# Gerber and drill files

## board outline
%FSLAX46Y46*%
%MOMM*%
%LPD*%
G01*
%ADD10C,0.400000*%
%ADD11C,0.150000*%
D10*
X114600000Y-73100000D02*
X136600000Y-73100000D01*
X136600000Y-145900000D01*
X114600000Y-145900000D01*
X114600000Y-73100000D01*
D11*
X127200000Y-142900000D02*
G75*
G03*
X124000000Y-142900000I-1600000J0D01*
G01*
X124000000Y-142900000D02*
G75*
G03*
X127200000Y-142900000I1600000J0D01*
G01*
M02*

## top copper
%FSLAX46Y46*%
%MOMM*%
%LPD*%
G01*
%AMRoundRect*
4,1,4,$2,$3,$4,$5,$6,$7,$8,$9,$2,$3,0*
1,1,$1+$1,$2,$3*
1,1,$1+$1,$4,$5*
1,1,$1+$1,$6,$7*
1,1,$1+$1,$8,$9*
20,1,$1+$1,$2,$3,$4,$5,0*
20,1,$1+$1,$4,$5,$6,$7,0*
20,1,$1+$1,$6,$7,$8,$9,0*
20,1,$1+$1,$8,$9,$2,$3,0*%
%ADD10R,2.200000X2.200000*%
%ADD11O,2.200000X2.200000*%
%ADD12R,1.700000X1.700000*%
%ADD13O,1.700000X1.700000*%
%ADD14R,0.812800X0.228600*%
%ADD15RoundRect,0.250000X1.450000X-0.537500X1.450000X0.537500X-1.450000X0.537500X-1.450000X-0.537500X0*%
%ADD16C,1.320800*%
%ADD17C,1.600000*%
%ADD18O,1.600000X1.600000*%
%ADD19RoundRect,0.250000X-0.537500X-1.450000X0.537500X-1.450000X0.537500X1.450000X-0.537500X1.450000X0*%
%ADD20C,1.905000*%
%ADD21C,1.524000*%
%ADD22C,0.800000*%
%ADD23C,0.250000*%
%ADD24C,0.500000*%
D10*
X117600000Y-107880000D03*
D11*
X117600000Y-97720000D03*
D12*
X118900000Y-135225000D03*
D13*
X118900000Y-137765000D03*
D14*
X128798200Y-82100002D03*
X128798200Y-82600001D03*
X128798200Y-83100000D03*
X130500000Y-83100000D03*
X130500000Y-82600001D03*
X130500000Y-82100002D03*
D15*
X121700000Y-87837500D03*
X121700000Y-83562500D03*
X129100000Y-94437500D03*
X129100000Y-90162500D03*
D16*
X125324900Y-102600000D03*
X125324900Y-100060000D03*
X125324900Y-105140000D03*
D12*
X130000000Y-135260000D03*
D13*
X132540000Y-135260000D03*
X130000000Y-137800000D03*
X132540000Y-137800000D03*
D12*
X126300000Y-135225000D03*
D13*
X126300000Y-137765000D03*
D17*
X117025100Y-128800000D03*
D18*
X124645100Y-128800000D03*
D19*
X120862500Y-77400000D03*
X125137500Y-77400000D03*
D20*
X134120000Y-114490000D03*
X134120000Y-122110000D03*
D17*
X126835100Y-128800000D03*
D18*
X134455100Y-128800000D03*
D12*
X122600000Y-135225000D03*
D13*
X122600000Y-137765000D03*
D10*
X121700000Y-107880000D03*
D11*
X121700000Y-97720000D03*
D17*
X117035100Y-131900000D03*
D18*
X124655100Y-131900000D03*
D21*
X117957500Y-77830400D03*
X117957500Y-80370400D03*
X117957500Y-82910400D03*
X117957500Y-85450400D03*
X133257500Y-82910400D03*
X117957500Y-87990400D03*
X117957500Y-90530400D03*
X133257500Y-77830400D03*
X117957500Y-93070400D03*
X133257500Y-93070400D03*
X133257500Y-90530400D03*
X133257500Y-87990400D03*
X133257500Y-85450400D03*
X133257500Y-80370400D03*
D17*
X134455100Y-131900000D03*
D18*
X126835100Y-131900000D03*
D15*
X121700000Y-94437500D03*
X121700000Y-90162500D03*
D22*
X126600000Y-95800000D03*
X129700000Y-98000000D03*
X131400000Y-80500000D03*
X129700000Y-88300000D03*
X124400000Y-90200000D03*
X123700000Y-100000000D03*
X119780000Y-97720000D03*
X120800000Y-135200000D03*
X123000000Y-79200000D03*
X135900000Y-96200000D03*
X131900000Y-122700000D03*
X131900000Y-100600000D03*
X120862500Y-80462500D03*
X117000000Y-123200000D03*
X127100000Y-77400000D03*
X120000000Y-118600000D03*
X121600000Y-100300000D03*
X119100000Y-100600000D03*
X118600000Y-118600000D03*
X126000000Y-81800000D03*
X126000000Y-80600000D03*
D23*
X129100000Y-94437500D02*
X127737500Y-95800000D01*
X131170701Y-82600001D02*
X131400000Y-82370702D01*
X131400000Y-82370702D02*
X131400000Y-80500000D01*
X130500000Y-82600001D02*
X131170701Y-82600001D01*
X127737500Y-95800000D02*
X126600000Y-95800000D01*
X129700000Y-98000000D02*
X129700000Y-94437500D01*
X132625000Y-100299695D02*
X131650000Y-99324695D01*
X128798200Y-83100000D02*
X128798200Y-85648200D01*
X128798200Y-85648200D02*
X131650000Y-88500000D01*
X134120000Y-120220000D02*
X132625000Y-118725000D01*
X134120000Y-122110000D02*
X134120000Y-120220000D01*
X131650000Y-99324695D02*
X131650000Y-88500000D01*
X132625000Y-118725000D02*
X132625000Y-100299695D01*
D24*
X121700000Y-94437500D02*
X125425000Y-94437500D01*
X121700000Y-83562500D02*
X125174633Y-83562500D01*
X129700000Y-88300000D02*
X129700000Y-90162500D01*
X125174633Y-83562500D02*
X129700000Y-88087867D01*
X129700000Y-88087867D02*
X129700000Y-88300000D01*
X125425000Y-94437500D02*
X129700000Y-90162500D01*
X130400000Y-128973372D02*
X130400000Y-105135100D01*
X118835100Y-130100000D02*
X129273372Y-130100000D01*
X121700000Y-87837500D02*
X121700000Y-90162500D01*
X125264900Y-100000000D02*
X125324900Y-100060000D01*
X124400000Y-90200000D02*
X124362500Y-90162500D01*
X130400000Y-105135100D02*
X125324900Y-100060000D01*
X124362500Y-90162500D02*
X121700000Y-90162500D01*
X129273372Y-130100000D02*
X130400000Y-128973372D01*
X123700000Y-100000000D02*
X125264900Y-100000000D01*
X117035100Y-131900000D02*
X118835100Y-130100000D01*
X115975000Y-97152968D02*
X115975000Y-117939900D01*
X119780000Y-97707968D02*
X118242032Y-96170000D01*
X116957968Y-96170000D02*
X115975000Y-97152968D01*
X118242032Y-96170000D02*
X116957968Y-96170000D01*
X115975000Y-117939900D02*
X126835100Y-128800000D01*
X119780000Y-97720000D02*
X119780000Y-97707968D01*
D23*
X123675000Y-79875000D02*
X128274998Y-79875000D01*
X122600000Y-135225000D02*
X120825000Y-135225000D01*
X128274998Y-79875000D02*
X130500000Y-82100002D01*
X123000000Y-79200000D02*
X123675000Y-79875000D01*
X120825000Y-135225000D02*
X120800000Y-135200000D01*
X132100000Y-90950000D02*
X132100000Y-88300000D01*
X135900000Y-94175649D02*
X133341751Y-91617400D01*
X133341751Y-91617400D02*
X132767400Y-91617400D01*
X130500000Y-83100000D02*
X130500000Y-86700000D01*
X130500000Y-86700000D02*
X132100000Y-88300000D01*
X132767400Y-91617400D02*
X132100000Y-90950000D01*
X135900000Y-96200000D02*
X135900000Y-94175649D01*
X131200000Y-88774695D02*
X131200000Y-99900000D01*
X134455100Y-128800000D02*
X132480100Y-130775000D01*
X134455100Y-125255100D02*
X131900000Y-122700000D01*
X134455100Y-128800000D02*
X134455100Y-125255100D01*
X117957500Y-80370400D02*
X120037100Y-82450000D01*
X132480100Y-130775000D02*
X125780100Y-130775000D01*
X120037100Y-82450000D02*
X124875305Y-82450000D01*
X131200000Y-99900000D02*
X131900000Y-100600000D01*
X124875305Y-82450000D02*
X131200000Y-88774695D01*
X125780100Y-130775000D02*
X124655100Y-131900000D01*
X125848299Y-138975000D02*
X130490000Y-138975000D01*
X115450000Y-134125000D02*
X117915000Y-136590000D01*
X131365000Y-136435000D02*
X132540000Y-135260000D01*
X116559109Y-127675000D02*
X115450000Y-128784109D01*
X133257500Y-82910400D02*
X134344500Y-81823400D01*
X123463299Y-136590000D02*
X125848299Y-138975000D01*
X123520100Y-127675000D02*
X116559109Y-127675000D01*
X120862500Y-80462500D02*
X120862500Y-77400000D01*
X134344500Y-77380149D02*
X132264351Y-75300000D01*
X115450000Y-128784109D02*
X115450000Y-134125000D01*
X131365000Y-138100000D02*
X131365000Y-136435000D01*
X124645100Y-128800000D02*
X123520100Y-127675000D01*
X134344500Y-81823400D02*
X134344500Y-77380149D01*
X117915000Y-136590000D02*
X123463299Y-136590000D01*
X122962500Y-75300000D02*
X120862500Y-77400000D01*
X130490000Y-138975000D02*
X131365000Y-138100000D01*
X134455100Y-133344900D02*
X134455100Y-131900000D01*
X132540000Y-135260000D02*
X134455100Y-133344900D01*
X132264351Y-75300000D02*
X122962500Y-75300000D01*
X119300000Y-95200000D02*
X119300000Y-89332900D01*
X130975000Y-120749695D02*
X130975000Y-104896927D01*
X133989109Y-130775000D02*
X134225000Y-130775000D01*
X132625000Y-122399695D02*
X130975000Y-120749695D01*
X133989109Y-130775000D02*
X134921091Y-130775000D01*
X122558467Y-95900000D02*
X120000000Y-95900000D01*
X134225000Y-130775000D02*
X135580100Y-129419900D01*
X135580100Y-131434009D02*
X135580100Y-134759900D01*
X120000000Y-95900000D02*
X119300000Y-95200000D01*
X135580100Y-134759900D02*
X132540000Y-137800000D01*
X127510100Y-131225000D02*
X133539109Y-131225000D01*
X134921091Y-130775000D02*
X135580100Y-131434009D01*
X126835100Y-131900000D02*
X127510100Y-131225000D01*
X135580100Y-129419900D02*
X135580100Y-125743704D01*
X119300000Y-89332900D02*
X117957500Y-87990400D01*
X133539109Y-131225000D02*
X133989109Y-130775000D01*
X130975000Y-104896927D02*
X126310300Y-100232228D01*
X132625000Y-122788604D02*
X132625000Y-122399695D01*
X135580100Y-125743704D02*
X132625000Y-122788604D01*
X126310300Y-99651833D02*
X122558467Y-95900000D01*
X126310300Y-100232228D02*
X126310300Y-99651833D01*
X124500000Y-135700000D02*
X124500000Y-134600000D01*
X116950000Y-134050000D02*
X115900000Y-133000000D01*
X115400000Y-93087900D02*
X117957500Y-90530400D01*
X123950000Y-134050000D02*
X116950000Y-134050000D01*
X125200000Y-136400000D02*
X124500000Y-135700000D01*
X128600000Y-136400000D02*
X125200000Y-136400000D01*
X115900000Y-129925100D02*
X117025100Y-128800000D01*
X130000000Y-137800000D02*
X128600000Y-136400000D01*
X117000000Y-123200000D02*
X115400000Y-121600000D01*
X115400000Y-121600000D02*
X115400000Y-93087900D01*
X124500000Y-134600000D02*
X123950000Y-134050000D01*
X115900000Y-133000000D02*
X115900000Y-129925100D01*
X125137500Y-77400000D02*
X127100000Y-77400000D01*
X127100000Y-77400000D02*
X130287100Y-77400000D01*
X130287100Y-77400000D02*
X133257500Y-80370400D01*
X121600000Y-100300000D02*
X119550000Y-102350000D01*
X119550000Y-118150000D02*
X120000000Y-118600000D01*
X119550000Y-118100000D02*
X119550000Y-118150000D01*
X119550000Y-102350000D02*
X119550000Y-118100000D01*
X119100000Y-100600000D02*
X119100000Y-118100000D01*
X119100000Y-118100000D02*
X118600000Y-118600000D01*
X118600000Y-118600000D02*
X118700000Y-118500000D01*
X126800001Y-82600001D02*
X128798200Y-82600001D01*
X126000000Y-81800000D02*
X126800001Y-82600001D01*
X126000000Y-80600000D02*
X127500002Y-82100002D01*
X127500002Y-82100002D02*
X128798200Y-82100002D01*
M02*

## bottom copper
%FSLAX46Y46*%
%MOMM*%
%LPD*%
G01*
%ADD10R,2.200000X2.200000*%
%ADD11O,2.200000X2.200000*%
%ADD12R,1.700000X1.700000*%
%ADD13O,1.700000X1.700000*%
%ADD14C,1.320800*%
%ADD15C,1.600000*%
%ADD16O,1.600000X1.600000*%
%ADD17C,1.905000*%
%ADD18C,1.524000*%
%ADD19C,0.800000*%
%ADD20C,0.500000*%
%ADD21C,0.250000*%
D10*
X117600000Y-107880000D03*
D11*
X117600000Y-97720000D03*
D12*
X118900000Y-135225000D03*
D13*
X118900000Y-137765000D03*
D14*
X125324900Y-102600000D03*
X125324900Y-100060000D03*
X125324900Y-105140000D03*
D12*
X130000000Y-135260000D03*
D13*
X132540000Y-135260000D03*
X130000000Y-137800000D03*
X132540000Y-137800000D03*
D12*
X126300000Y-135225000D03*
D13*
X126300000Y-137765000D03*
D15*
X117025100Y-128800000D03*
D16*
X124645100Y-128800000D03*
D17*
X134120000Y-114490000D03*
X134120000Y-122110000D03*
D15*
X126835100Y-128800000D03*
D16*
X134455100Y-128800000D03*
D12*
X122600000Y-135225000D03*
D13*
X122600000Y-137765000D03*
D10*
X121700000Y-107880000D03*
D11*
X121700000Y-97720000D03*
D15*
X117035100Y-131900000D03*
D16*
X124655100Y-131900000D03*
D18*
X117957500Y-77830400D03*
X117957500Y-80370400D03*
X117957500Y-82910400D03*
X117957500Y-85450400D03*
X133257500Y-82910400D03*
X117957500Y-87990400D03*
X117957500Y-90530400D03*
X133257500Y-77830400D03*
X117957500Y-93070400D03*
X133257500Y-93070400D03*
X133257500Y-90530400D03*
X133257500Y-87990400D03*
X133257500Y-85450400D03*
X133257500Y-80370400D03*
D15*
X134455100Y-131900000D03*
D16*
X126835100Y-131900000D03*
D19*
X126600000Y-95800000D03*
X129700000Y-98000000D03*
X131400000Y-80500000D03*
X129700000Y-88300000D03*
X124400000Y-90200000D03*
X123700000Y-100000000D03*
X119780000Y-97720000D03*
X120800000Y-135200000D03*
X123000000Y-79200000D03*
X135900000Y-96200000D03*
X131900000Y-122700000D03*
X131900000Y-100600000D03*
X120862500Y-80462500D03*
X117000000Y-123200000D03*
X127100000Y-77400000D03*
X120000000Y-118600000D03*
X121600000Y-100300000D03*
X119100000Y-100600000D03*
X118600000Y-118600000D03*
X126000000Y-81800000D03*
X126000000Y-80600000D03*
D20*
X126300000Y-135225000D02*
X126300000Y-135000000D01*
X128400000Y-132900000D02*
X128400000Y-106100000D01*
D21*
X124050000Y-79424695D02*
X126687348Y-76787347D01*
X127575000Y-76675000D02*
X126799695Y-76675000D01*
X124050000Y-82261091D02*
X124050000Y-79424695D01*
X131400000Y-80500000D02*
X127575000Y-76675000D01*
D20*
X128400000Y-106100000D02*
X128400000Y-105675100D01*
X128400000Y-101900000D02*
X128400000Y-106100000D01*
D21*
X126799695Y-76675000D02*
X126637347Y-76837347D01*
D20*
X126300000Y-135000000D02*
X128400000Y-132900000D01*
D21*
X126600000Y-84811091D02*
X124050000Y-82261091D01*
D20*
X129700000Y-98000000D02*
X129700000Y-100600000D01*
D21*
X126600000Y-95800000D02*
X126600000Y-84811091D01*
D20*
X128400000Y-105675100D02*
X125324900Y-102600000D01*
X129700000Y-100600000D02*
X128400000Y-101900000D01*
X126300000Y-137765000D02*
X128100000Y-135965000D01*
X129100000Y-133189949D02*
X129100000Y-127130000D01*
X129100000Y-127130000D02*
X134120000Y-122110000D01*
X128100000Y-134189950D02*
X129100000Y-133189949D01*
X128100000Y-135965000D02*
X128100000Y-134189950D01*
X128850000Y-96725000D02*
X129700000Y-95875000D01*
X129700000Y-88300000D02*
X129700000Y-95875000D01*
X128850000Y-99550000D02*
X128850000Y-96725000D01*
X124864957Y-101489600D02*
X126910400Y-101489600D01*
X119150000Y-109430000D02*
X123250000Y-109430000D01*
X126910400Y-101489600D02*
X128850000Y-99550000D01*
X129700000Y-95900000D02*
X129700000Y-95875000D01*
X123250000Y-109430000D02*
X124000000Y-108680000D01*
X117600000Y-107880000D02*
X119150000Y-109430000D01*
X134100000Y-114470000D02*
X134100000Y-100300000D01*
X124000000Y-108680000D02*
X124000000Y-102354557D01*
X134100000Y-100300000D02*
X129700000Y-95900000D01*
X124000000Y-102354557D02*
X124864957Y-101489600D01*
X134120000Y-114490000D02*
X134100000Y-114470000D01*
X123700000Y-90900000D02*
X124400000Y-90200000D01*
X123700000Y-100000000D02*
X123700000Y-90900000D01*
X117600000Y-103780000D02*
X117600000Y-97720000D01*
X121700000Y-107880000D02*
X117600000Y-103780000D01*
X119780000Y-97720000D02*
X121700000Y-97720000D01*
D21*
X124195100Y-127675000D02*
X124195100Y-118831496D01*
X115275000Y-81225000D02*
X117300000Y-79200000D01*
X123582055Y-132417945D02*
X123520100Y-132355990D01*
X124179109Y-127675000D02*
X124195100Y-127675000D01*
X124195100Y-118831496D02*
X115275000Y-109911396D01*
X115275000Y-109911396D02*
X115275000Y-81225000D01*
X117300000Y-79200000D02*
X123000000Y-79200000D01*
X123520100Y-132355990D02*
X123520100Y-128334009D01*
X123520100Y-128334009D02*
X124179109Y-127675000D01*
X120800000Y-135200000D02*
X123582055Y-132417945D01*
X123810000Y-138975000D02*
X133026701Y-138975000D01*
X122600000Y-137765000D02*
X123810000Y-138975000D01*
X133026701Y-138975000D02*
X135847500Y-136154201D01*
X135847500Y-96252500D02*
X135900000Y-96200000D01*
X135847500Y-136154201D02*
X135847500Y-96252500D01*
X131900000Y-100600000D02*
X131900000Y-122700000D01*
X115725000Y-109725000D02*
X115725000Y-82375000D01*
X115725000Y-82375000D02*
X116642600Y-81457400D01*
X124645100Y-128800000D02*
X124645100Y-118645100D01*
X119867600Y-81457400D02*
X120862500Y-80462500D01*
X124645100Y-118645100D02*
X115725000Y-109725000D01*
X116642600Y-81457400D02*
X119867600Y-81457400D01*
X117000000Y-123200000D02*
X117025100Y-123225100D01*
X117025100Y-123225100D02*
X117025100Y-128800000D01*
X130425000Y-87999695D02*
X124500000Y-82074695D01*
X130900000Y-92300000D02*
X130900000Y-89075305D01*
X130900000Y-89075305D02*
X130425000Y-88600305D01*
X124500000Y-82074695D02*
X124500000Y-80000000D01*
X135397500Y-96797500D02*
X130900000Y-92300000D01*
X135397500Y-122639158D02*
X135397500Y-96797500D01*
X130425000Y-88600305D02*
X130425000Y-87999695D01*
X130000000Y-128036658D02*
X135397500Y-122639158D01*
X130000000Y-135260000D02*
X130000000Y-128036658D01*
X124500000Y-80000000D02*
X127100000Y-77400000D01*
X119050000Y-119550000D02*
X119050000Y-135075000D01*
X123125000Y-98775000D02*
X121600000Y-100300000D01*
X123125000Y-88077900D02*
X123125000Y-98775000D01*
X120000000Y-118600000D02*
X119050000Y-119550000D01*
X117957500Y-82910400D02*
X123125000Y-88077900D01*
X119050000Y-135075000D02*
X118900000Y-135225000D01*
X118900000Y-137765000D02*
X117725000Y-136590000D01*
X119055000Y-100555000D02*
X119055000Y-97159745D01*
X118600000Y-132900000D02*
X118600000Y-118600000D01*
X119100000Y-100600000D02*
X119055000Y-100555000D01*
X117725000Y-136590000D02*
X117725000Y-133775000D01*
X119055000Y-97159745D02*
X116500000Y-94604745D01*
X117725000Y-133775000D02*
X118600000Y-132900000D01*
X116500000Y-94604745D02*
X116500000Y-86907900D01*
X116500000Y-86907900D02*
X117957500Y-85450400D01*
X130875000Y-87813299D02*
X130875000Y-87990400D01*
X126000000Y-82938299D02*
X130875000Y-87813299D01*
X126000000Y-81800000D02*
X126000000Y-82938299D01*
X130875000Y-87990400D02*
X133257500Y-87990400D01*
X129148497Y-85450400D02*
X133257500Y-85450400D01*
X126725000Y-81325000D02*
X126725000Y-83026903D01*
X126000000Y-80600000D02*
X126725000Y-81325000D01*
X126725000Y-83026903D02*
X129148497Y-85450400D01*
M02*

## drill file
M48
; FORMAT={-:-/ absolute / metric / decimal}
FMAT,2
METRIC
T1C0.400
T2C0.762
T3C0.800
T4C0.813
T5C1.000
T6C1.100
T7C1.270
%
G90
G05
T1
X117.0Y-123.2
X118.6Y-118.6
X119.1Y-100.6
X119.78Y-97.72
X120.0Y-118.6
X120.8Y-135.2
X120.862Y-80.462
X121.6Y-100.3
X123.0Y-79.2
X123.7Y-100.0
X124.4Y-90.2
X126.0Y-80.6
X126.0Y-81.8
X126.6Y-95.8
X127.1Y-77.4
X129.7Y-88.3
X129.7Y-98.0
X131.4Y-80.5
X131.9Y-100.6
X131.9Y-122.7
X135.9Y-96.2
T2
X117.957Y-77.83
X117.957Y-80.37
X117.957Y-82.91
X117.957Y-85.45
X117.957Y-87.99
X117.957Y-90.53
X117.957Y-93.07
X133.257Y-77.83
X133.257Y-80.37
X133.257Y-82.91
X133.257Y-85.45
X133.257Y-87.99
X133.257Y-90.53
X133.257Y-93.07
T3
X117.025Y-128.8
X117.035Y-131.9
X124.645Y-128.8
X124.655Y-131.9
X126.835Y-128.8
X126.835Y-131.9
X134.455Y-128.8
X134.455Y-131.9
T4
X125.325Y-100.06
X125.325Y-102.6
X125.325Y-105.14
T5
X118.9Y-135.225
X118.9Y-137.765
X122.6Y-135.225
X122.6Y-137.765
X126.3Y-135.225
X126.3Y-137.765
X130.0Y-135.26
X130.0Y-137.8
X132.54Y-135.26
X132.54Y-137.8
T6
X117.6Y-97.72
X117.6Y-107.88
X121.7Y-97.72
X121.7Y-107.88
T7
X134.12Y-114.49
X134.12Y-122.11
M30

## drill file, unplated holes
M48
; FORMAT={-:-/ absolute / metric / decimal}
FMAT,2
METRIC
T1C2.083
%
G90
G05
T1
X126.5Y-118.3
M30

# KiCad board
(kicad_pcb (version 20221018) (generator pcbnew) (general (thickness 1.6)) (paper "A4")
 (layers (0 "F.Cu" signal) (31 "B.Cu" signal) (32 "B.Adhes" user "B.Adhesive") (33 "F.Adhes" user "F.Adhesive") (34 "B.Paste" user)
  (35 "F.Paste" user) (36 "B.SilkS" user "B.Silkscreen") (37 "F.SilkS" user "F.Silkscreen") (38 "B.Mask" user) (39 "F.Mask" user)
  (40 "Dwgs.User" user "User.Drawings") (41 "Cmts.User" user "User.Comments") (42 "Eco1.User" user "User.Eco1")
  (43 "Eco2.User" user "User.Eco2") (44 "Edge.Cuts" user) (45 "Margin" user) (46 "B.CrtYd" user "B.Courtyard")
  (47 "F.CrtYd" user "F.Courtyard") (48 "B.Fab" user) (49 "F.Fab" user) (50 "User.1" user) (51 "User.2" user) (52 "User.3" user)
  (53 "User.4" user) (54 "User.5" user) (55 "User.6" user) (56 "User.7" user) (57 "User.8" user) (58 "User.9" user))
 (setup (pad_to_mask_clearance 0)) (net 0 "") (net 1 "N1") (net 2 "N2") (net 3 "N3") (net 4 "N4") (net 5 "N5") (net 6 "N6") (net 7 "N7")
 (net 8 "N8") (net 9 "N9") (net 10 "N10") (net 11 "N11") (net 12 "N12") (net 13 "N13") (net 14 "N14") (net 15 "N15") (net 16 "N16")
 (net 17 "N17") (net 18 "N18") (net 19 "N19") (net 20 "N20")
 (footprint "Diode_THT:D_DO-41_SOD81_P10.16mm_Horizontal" (layer "F.Cu") (at 117.6 107.88 90)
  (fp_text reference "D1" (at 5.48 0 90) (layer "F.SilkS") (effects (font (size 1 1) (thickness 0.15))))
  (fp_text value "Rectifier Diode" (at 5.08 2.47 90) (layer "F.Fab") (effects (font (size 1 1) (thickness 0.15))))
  (pad "1" thru_hole rect (at 0 0 90) (size 2.2 2.2) (drill 1.1) (layers "*.Cu" "*.Mask") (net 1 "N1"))
  (pad "2" thru_hole oval (at 10.16 0 90) (size 2.2 2.2) (drill 1.1) (layers "*.Cu" "*.Mask") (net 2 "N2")))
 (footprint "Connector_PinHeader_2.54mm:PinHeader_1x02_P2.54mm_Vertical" (layer "F.Cu") (at 118.9 135.225)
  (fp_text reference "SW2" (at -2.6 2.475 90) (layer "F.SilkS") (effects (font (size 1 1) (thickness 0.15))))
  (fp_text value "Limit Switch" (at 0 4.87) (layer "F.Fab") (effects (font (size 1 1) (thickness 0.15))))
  (pad "1" thru_hole rect (at 0 0) (size 1.7 1.7) (drill 1) (layers "*.Cu" "*.Mask") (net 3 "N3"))
  (pad "2" thru_hole oval (at 0 2.54) (size 1.7 1.7) (drill 1) (layers "*.Cu" "*.Mask") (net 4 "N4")))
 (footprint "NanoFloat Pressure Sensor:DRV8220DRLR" (layer "F.Cu") (at 129.6491 82.600001)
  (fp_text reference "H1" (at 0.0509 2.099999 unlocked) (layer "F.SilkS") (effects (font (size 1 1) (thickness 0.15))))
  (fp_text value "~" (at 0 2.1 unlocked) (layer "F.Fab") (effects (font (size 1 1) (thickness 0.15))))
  (pad "1" smd rect (at -0.8509 -0.499999) (size 0.8128 0.2286) (layers "F.Cu" "F.Paste" "F.Mask") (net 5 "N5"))
  (pad "2" smd rect (at -0.8509 0) (size 0.8128 0.2286) (layers "F.Cu" "F.Paste" "F.Mask") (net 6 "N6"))
  (pad "3" smd rect (at -0.8509 0.499999) (size 0.8128 0.2286) (layers "F.Cu" "F.Paste" "F.Mask") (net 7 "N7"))
  (pad "4" smd rect (at 0.8509 0.499999) (size 0.8128 0.2286) (layers "F.Cu" "F.Paste" "F.Mask") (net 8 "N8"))
  (pad "5" smd rect (at 0.8509 0) (size 0.8128 0.2286) (layers "F.Cu" "F.Paste" "F.Mask") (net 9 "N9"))
  (pad "6" smd rect (at 0.8509 -0.499999) (size 0.8128 0.2286) (layers "F.Cu" "F.Paste" "F.Mask") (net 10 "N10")))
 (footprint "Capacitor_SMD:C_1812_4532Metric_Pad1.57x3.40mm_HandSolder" (layer "F.Cu") (at 121.7 85.7 90)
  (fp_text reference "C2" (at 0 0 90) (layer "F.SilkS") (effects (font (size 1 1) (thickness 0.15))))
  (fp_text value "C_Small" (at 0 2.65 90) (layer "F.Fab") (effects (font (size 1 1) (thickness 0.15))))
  (pad "1" smd roundrect (at -2.1375 0 90) (size 1.575 3.4) (layers "F.Cu" "F.Paste" "F.Mask") (roundrect_rratio 0.1587301587)
   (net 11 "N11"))
  (pad "2" smd roundrect (at 2.1375 0 90) (size 1.575 3.4) (layers "F.Cu" "F.Paste" "F.Mask") (roundrect_rratio 0.1587301587) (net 1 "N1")))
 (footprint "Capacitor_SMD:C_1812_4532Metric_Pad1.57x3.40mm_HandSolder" (layer "F.Cu") (at 129.1 92.3 90)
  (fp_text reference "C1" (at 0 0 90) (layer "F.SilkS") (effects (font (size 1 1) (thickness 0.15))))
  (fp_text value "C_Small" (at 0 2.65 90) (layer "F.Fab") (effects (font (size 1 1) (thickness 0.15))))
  (pad "1" smd roundrect (at -2.1375 0 90) (size 1.575 3.4) (layers "F.Cu" "F.Paste" "F.Mask") (roundrect_rratio 0.1587301587) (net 9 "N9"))
  (pad "2" smd roundrect (at 2.1375 0 90) (size 1.575 3.4) (layers "F.Cu" "F.Paste" "F.Mask") (roundrect_rratio 0.1587301587) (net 1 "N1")))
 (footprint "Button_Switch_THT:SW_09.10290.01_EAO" (layer "F.Cu") (at 125.3249 102.6 90)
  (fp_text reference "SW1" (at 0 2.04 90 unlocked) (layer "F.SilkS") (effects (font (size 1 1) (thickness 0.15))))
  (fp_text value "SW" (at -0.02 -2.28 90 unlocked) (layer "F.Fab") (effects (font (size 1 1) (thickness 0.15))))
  (pad "1" thru_hole circle (at 0 0 90) (size 1.3208 1.3208) (drill 0.8128) (layers "*.Cu" "*.Mask") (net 9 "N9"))
  (pad "2" thru_hole circle (at 2.54 0 90) (size 1.3208 1.3208) (drill 0.8128) (layers "*.Cu" "*.Mask") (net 11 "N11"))
  (pad "3" thru_hole circle (at -2.54 0 90) (size 1.3208 1.3208) (drill 0.8128) (layers "*.Cu" "*.Mask") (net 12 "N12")))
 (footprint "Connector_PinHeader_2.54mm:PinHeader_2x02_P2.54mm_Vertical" (layer "F.Cu") (at 130 135.26)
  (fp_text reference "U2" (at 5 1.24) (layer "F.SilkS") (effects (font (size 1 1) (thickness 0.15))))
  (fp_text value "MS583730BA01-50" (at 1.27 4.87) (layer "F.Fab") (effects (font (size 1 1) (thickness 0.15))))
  (pad "1" thru_hole rect (at 0 0) (size 1.7 1.7) (drill 1) (layers "*.Cu" "*.Mask") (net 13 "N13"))
  (pad "2" thru_hole oval (at 2.54 0) (size 1.7 1.7) (drill 1) (layers "*.Cu" "*.Mask") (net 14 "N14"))
  (pad "3" thru_hole oval (at 0 2.54) (size 1.7 1.7) (drill 1) (layers "*.Cu" "*.Mask") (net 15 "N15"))
  (pad "4" thru_hole oval (at 2.54 2.54) (size 1.7 1.7) (drill 1) (layers "*.Cu" "*.Mask") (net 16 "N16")))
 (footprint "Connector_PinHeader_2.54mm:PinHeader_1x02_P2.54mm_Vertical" (layer "F.Cu") (at 126.3 135.225)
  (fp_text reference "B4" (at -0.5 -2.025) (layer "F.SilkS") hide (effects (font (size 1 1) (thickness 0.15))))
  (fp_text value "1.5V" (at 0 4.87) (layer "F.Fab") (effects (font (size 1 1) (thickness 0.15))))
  (pad "1" thru_hole rect (at 0 0) (size 1.7 1.7) (drill 1) (layers "*.Cu" "*.Mask") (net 9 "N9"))
  (pad "2" thru_hole oval (at 0 2.54) (size 1.7 1.7) (drill 1) (layers "*.Cu" "*.Mask") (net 7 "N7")))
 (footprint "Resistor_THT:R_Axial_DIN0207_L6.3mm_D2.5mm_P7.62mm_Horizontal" (layer "F.Cu") (at 117.0251 128.8)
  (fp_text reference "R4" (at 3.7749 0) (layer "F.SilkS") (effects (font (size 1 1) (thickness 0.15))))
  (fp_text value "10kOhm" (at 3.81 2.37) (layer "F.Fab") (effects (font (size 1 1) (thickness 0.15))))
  (pad "1" thru_hole circle (at 0 0) (size 1.6 1.6) (drill 0.8) (layers "*.Cu" "*.Mask") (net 15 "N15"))
  (pad "2" thru_hole oval (at 7.62 0) (size 1.6 1.6) (drill 0.8) (layers "*.Cu" "*.Mask") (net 14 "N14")))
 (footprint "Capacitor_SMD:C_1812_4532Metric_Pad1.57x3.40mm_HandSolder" (layer "F.Cu") (at 123 77.4)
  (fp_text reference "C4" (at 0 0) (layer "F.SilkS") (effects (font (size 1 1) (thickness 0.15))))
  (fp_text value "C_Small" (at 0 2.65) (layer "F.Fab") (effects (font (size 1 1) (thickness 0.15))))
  (pad "1" smd roundrect (at -2.1375 0) (size 1.575 3.4) (layers "F.Cu" "F.Paste" "F.Mask") (roundrect_rratio 0.1587301587) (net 14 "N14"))
  (pad "2" smd roundrect (at 2.1375 0) (size 1.575 3.4) (layers "F.Cu" "F.Paste" "F.Mask") (roundrect_rratio 0.1587301587) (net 13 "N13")))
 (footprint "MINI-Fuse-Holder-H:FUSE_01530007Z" (layer "F.Cu") (at 126.5 118.3 -90)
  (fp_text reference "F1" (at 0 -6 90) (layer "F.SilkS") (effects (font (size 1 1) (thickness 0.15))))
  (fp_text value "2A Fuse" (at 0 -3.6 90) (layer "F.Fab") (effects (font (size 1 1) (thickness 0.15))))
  (pad "" np_thru_hole circle (at 0 0 270) (size 2.0828 2.0828) (drill 2.0828) (layers "*.Cu" "*.Mask"))
  (pad "1" thru_hole circle (at -3.81 -7.62 270) (size 1.905 1.905) (drill 1.27) (layers "*.Cu" "*.Mask") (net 1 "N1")
   (solder_mask_margin 0.102))
  (pad "2" thru_hole circle (at 3.81 -7.62 270) (size 1.905 1.905) (drill 1.27) (layers "*.Cu" "*.Mask") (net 7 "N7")
   (solder_mask_margin 0.102)))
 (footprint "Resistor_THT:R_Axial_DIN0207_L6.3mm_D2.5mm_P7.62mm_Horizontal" (layer "F.Cu") (at 126.8351 128.8)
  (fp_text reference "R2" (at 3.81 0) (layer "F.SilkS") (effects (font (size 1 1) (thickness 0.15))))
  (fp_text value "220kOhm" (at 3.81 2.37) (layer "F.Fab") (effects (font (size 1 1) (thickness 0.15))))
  (pad "1" thru_hole circle (at 0 0) (size 1.6 1.6) (drill 0.8) (layers "*.Cu" "*.Mask") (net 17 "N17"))
  (pad "2" thru_hole oval (at 7.62 0) (size 1.6 1.6) (drill 0.8) (layers "*.Cu" "*.Mask") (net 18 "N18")))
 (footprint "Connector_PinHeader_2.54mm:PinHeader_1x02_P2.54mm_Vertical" (layer "F.Cu") (at 122.6 135.225)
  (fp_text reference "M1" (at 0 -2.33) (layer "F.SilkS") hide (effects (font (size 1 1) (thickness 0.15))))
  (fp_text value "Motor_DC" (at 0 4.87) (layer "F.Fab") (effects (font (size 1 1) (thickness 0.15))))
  (pad "1" thru_hole rect (at 0 0) (size 1.7 1.7) (drill 1) (layers "*.Cu" "*.Mask") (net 10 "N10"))
  (pad "2" thru_hole oval (at 0 2.54) (size 1.7 1.7) (drill 1) (layers "*.Cu" "*.Mask") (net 8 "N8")))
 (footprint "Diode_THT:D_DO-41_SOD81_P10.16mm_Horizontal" (layer "F.Cu") (at 121.7 107.88 90)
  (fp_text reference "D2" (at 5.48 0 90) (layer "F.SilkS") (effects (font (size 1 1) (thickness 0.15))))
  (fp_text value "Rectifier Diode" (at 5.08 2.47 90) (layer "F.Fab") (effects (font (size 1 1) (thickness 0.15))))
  (pad "1" thru_hole rect (at 0 0 90) (size 2.2 2.2) (drill 1.1) (layers "*.Cu" "*.Mask") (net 2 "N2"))
  (pad "2" thru_hole oval (at 10.16 0 90) (size 2.2 2.2) (drill 1.1) (layers "*.Cu" "*.Mask") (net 17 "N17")))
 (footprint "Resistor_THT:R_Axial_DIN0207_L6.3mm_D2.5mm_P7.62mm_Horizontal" (layer "F.Cu") (at 117.0351 131.9)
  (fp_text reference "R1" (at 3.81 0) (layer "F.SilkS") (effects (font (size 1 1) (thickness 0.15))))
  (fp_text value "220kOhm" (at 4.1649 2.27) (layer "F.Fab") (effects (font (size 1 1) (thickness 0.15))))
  (pad "1" thru_hole circle (at 0 0) (size 1.6 1.6) (drill 0.8) (layers "*.Cu" "*.Mask") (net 11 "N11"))
  (pad "2" thru_hole oval (at 7.62 0) (size 1.6 1.6) (drill 0.8) (layers "*.Cu" "*.Mask") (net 18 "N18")))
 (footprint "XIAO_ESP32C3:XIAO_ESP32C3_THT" (layer "F.Cu") (at 125.5575 87.8704)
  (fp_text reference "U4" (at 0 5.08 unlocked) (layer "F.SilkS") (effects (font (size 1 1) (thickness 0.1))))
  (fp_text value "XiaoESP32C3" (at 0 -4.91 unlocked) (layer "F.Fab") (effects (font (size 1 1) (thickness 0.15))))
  (pad "0" thru_hole circle (at -7.6 -10.04) (size 1.524 1.524) (drill 0.762) (layers "*.Cu" "*.Mask"))
  (pad "1" thru_hole circle (at -7.6 -7.5) (size 1.524 1.524) (drill 0.762) (layers "*.Cu" "*.Mask") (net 18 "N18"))
  (pad "2" thru_hole circle (at -7.6 -4.96) (size 1.524 1.524) (drill 0.762) (layers "*.Cu" "*.Mask") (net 3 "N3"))
  (pad "3" thru_hole circle (at -7.6 -2.42) (size 1.524 1.524) (drill 0.762) (layers "*.Cu" "*.Mask") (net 4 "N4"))
  (pad "3V3" thru_hole circle (at 7.7 -4.96) (size 1.524 1.524) (drill 0.762) (layers "*.Cu" "*.Mask") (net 14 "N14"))
  (pad "4" thru_hole circle (at -7.6 0.12) (size 1.524 1.524) (drill 0.762) (layers "*.Cu" "*.Mask") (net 16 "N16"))
  (pad "5" thru_hole circle (at -7.6 2.66) (size 1.524 1.524) (drill 0.762) (layers "*.Cu" "*.Mask") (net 15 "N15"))
  (pad "5V" thru_hole circle (at 7.7 -10.04) (size 1.524 1.524) (drill 0.762) (layers "*.Cu" "*.Mask"))
  (pad "6" thru_hole circle (at -7.6 5.2) (size 1.524 1.524) (drill 0.762) (layers "*.Cu" "*.Mask"))
  (pad "7" thru_hole circle (at 7.7 5.2) (size 1.524 1.524) (drill 0.762) (layers "*.Cu" "*.Mask") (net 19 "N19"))
  (pad "8" thru_hole circle (at 7.7 2.66) (size 1.524 1.524) (drill 0.762) (layers "*.Cu" "*.Mask") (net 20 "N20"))
  (pad "9" thru_hole circle (at 7.7 0.12) (size 1.524 1.524) (drill 0.762) (layers "*.Cu" "*.Mask") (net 6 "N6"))
  (pad "10" thru_hole circle (at 7.7 -2.42) (size 1.524 1.524) (drill 0.762) (layers "*.Cu" "*.Mask") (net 5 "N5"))
  (pad "GND" thru_hole circle (at 7.7 -7.5) (size 1.524 1.524) (drill 0.762) (layers "*.Cu" "*.Mask") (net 13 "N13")))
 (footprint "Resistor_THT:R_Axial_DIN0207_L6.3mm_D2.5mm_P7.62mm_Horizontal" (layer "F.Cu") (at 134.4551 131.9 180)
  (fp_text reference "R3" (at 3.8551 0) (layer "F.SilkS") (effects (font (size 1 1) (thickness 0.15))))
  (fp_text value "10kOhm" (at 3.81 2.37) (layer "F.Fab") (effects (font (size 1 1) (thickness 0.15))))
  (pad "1" thru_hole circle (at 0 0 180) (size 1.6 1.6) (drill 0.8) (layers "*.Cu" "*.Mask") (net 14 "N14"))
  (pad "2" thru_hole oval (at 7.62 0 180) (size 1.6 1.6) (drill 0.8) (layers "*.Cu" "*.Mask") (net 16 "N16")))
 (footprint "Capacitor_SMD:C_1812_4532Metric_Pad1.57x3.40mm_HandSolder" (layer "F.Cu") (at 121.7 92.3 90)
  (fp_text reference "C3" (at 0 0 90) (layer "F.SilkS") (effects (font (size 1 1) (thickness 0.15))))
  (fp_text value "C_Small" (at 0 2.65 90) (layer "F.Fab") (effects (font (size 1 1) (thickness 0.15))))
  (pad "1" smd roundrect (at -2.1375 0 90) (size 1.575 3.4) (layers "F.Cu" "F.Paste" "F.Mask") (roundrect_rratio 0.1587301587) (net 1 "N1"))
  (pad "2" smd roundrect (at 2.1375 0 90) (size 1.575 3.4) (layers "F.Cu" "F.Paste" "F.Mask") (roundrect_rratio 0.1587301587) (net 11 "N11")))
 (gr_rect (start 114.6 73.1) (end 136.6 145.9) (stroke (width 0.4) (type default)) (fill none) (layer "Edge.Cuts"))
 (gr_circle (center 125.6 142.9) (end 127.2 142.9) (stroke (width 0.15) (type default)) (fill none) (layer "Edge.Cuts"))
 (segment (start 129.1 94.4375) (end 127.7375 95.8) (width 0.25) (layer "F.Cu") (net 9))
 (segment (start 131.170701 82.600001) (end 131.4 82.370702) (width 0.25) (layer "F.Cu") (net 9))
 (segment (start 131.4 82.370702) (end 131.4 80.5) (width 0.25) (layer "F.Cu") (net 9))
 (segment (start 130.5 82.600001) (end 131.170701 82.600001) (width 0.25) (layer "F.Cu") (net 9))
 (segment (start 127.7375 95.8) (end 126.6 95.8) (width 0.25) (layer "F.Cu") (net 9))
 (segment (start 129.7 98) (end 129.7 94.4375) (width 0.25) (layer "F.Cu") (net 9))
 (via (at 126.6 95.8) (size 0.8) (drill 0.4) (layers "F.Cu" "B.Cu") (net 9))
 (via (at 129.7 98) (size 0.8) (drill 0.4) (layers "F.Cu" "B.Cu") (free) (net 9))
 (via (at 131.4 80.5) (size 0.8) (drill 0.4) (layers "F.Cu" "B.Cu") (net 9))
 (segment (start 126.3 135.225) (end 126.3 135) (width 0.5) (layer "B.Cu") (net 9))
 (segment (start 128.4 132.9) (end 128.4 106.1) (width 0.5) (layer "B.Cu") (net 9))
 (segment (start 124.05 79.424695) (end 126.687348 76.787347) (width 0.25) (layer "B.Cu") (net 9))
 (segment (start 127.575 76.675) (end 126.799695 76.675) (width 0.25) (layer "B.Cu") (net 9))
 (segment (start 124.05 82.261091) (end 124.05 79.424695) (width 0.25) (layer "B.Cu") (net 9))
 (segment (start 131.4 80.5) (end 127.575 76.675) (width 0.25) (layer "B.Cu") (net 9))
 (segment (start 128.4 106.1) (end 128.4 105.6751) (width 0.5) (layer "B.Cu") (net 9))
 (segment (start 128.4 101.9) (end 128.4 106.1) (width 0.5) (layer "B.Cu") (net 9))
 (segment (start 126.799695 76.675) (end 126.637347 76.837347) (width 0.25) (layer "B.Cu") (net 9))
 (segment (start 126.3 135) (end 128.4 132.9) (width 0.5) (layer "B.Cu") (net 9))
 (segment (start 126.6 84.811091) (end 124.05 82.261091) (width 0.25) (layer "B.Cu") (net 9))
 (segment (start 129.7 98) (end 129.7 100.6) (width 0.5) (layer "B.Cu") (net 9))
 (segment (start 126.6 95.8) (end 126.6 84.811091) (width 0.25) (layer "B.Cu") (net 9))
 (segment (start 128.4 105.6751) (end 125.3249 102.6) (width 0.5) (layer "B.Cu") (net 9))
 (segment (start 129.7 100.6) (end 128.4 101.9) (width 0.5) (layer "B.Cu") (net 9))
 (segment (start 132.625 100.299695) (end 131.65 99.324695) (width 0.25) (layer "F.Cu") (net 7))
 (segment (start 128.7982 83.1) (end 128.7982 85.6482) (width 0.25) (layer "F.Cu") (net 7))
 (segment (start 128.7982 85.6482) (end 131.65 88.5) (width 0.25) (layer "F.Cu") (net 7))
 (segment (start 134.12 120.22) (end 132.625 118.725) (width 0.25) (layer "F.Cu") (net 7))
 (segment (start 134.12 122.11) (end 134.12 120.22) (width 0.25) (layer "F.Cu") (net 7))
 (segment (start 131.65 99.324695) (end 131.65 88.5) (width 0.25) (layer "F.Cu") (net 7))
 (segment (start 132.625 118.725) (end 132.625 100.299695) (width 0.25) (layer "F.Cu") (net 7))
 (segment (start 126.3 137.765) (end 128.1 135.965) (width 0.5) (layer "B.Cu") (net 7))
 (segment (start 129.1 133.189949) (end 129.1 127.13) (width 0.5) (layer "B.Cu") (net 7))
 (segment (start 129.1 127.13) (end 134.12 122.11) (width 0.5) (layer "B.Cu") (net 7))
 (segment (start 128.1 134.18995) (end 129.1 133.189949) (width 0.5) (layer "B.Cu") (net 7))
 (segment (start 128.1 135.965) (end 128.1 134.18995) (width 0.5) (layer "B.Cu") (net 7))
 (segment (start 121.7 94.4375) (end 125.425 94.4375) (width 0.5) (layer "F.Cu") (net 1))
 (segment (start 121.7 83.5625) (end 125.174633 83.5625) (width 0.5) (layer "F.Cu") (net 1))
 (segment (start 129.7 88.3) (end 129.7 90.1625) (width 0.5) (layer "F.Cu") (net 1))
 (segment (start 125.174633 83.5625) (end 129.7 88.087867) (width 0.5) (layer "F.Cu") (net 1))
 (segment (start 129.7 88.087867) (end 129.7 88.3) (width 0.5) (layer "F.Cu") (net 1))
 (segment (start 125.425 94.4375) (end 129.7 90.1625) (width 0.5) (layer "F.Cu") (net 1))
 (via (at 129.7 88.3) (size 0.8) (drill 0.4) (layers "F.Cu" "B.Cu") (free) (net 1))
 (segment (start 128.85 96.725) (end 129.7 95.875) (width 0.5) (layer "B.Cu") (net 1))
 (segment (start 129.7 88.3) (end 129.7 95.875) (width 0.5) (layer "B.Cu") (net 1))
 (segment (start 128.85 99.55) (end 128.85 96.725) (width 0.5) (layer "B.Cu") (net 1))
 (segment (start 124.864957 101.4896) (end 126.9104 101.4896) (width 0.5) (layer "B.Cu") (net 1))
 (segment (start 119.15 109.43) (end 123.25 109.43) (width 0.5) (layer "B.Cu") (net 1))
 (segment (start 126.9104 101.4896) (end 128.85 99.55) (width 0.5) (layer "B.Cu") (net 1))
 (segment (start 129.7 95.9) (end 129.7 95.875) (width 0.5) (layer "B.Cu") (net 1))
 (segment (start 123.25 109.43) (end 124 108.68) (width 0.5) (layer "B.Cu") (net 1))
 (segment (start 117.6 107.88) (end 119.15 109.43) (width 0.5) (layer "B.Cu") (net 1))
 (segment (start 134.1 114.47) (end 134.1 100.3) (width 0.5) (layer "B.Cu") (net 1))
 (segment (start 124 108.68) (end 124 102.354557) (width 0.5) (layer "B.Cu") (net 1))
 (segment (start 134.1 100.3) (end 129.7 95.9) (width 0.5) (layer "B.Cu") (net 1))
 (segment (start 124 102.354557) (end 124.864957 101.4896) (width 0.5) (layer "B.Cu") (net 1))
 (segment (start 134.12 114.49) (end 134.1 114.47) (width 0.5) (layer "B.Cu") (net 1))
 (segment (start 130.4 128.973372) (end 130.4 105.1351) (width 0.5) (layer "F.Cu") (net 11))
 (segment (start 118.8351 130.1) (end 129.273372 130.1) (width 0.5) (layer "F.Cu") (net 11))
 (segment (start 121.7 87.8375) (end 121.7 90.1625) (width 0.5) (layer "F.Cu") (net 11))
 (segment (start 125.2649 100) (end 125.3249 100.06) (width 0.5) (layer "F.Cu") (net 11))
 (segment (start 124.4 90.2) (end 124.3625 90.1625) (width 0.5) (layer "F.Cu") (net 11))
 (segment (start 130.4 105.1351) (end 125.3249 100.06) (width 0.5) (layer "F.Cu") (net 11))
 (segment (start 124.3625 90.1625) (end 121.7 90.1625) (width 0.5) (layer "F.Cu") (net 11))
 (segment (start 129.273372 130.1) (end 130.4 128.973372) (width 0.5) (layer "F.Cu") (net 11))
 (segment (start 123.7 100) (end 125.2649 100) (width 0.5) (layer "F.Cu") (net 11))
 (segment (start 117.0351 131.9) (end 118.8351 130.1) (width 0.5) (layer "F.Cu") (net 11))
 (via (at 124.4 90.2) (size 0.8) (drill 0.4) (layers "F.Cu" "B.Cu") (free) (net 11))
 (via (at 123.7 100) (size 0.8) (drill 0.4) (layers "F.Cu" "B.Cu") (free) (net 11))
 (segment (start 123.7 90.9) (end 124.4 90.2) (width 0.5) (layer "B.Cu") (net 11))
 (segment (start 123.7 100) (end 123.7 90.9) (width 0.5) (layer "B.Cu") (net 11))
 (segment (start 117.6 103.78) (end 117.6 97.72) (width 0.5) (layer "B.Cu") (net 2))
 (segment (start 121.7 107.88) (end 117.6 103.78) (width 0.5) (layer "B.Cu") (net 2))
 (segment (start 115.975 97.152968) (end 115.975 117.9399) (width 0.5) (layer "F.Cu") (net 17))
 (segment (start 119.78 97.707968) (end 118.242032 96.17) (width 0.5) (layer "F.Cu") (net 17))
 (segment (start 116.957968 96.17) (end 115.975 97.152968) (width 0.5) (layer "F.Cu") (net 17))
 (segment (start 118.242032 96.17) (end 116.957968 96.17) (width 0.5) (layer "F.Cu") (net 17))
 (segment (start 115.975 117.9399) (end 126.8351 128.8) (width 0.5) (layer "F.Cu") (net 17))
 (segment (start 119.78 97.72) (end 119.78 97.707968) (width 0.5) (layer "F.Cu") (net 17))
 (via (at 119.78 97.72) (size 0.8) (drill 0.4) (layers "F.Cu" "B.Cu") (free) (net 17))
 (segment (start 119.78 97.72) (end 121.7 97.72) (width 0.5) (layer "B.Cu") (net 17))
 (segment (start 123.675 79.875) (end 128.274998 79.875) (width 0.25) (layer "F.Cu") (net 10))
 (segment (start 122.6 135.225) (end 120.825 135.225) (width 0.25) (layer "F.Cu") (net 10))
 (segment (start 128.274998 79.875) (end 130.5 82.100002) (width 0.25) (layer "F.Cu") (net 10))
 (segment (start 123 79.2) (end 123.675 79.875) (width 0.25) (layer "F.Cu") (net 10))
 (segment (start 120.825 135.225) (end 120.8 135.2) (width 0.25) (layer "F.Cu") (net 10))
 (via (at 120.8 135.2) (size 0.8) (drill 0.4) (layers "F.Cu" "B.Cu") (free) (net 10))
 (via (at 123 79.2) (size 0.8) (drill 0.4) (layers "F.Cu" "B.Cu") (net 10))
 (segment (start 124.1951 127.675) (end 124.1951 118.831496) (width 0.25) (layer "B.Cu") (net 10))
 (segment (start 115.275 81.225) (end 117.3 79.2) (width 0.25) (layer "B.Cu") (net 10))
 (segment (start 123.582055 132.417945) (end 123.5201 132.35599) (width 0.25) (layer "B.Cu") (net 10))
 (segment (start 124.179109 127.675) (end 124.1951 127.675) (width 0.25) (layer "B.Cu") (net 10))
 (segment (start 124.1951 118.831496) (end 115.275 109.911396) (width 0.25) (layer "B.Cu") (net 10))
 (segment (start 115.275 109.911396) (end 115.275 81.225) (width 0.25) (layer "B.Cu") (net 10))
 (segment (start 117.3 79.2) (end 123 79.2) (width 0.25) (layer "B.Cu") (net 10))
 (segment (start 123.5201 132.35599) (end 123.5201 128.334009) (width 0.25) (layer "B.Cu") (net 10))
 (segment (start 123.5201 128.334009) (end 124.179109 127.675) (width 0.25) (layer "B.Cu") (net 10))
 (segment (start 120.8 135.2) (end 123.582055 132.417945) (width 0.25) (layer "B.Cu") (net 10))
 (segment (start 132.1 90.95) (end 132.1 88.3) (width 0.25) (layer "F.Cu") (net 8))
 (segment (start 135.9 94.175649) (end 133.341751 91.6174) (width 0.25) (layer "F.Cu") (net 8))
 (segment (start 133.341751 91.6174) (end 132.7674 91.6174) (width 0.25) (layer "F.Cu") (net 8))
 (segment (start 130.5 83.1) (end 130.5 86.7) (width 0.25) (layer "F.Cu") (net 8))
 (segment (start 130.5 86.7) (end 132.1 88.3) (width 0.25) (layer "F.Cu") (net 8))
 (segment (start 132.7674 91.6174) (end 132.1 90.95) (width 0.25) (layer "F.Cu") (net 8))
 (segment (start 135.9 96.2) (end 135.9 94.175649) (width 0.25) (layer "F.Cu") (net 8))
 (via (at 135.9 96.2) (size 0.8) (drill 0.4) (layers "F.Cu" "B.Cu") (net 8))
 (segment (start 123.81 138.975) (end 133.026701 138.975) (width 0.25) (layer "B.Cu") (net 8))
 (segment (start 122.6 137.765) (end 123.81 138.975) (width 0.25) (layer "B.Cu") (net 8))
 (segment (start 133.026701 138.975) (end 135.8475 136.154201) (width 0.25) (layer "B.Cu") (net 8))
 (segment (start 135.8475 96.2525) (end 135.9 96.2) (width 0.25) (layer "B.Cu") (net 8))
 (segment (start 135.8475 136.154201) (end 135.8475 96.2525) (width 0.25) (layer "B.Cu") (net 8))
 (segment (start 131.2 88.774695) (end 131.2 99.9) (width 0.25) (layer "F.Cu") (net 18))
 (segment (start 134.4551 128.8) (end 132.4801 130.775) (width 0.25) (layer "F.Cu") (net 18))
 (segment (start 134.4551 125.2551) (end 131.9 122.7) (width 0.25) (layer "F.Cu") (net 18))
 (segment (start 134.4551 128.8) (end 134.4551 125.2551) (width 0.25) (layer "F.Cu") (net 18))
 (segment (start 117.9575 80.3704) (end 120.0371 82.45) (width 0.25) (layer "F.Cu") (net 18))
 (segment (start 132.4801 130.775) (end 125.7801 130.775) (width 0.25) (layer "F.Cu") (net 18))
 (segment (start 120.0371 82.45) (end 124.875305 82.45) (width 0.25) (layer "F.Cu") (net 18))
 (segment (start 131.2 99.9) (end 131.9 100.6) (width 0.25) (layer "F.Cu") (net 18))
 (segment (start 124.875305 82.45) (end 131.2 88.774695) (width 0.25) (layer "F.Cu") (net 18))
 (segment (start 125.7801 130.775) (end 124.6551 131.9) (width 0.25) (layer "F.Cu") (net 18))
 (via (at 131.9 122.7) (size 0.8) (drill 0.4) (layers "F.Cu" "B.Cu") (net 18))
 (via (at 131.9 100.6) (size 0.8) (drill 0.4) (layers "F.Cu" "B.Cu") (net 18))
 (segment (start 131.9 100.6) (end 131.9 122.7) (width 0.25) (layer "B.Cu") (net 18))
 (segment (start 125.848299 138.975) (end 130.49 138.975) (width 0.25) (layer "F.Cu") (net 14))
 (segment (start 115.45 134.125) (end 117.915 136.59) (width 0.25) (layer "F.Cu") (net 14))
 (segment (start 131.365 136.435) (end 132.54 135.26) (width 0.25) (layer "F.Cu") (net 14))
 (segment (start 116.559109 127.675) (end 115.45 128.784109) (width 0.25) (layer "F.Cu") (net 14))
 (segment (start 133.2575 82.9104) (end 134.3445 81.8234) (width 0.25) (layer "F.Cu") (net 14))
 (segment (start 123.463299 136.59) (end 125.848299 138.975) (width 0.25) (layer "F.Cu") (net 14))
 (segment (start 123.5201 127.675) (end 116.559109 127.675) (width 0.25) (layer "F.Cu") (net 14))
 (segment (start 120.8625 80.4625) (end 120.8625 77.4) (width 0.25) (layer "F.Cu") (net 14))
 (segment (start 134.3445 77.380149) (end 132.264351 75.3) (width 0.25) (layer "F.Cu") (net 14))
 (segment (start 115.45 128.784109) (end 115.45 134.125) (width 0.25) (layer "F.Cu") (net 14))
 (segment (start 131.365 138.1) (end 131.365 136.435) (width 0.25) (layer "F.Cu") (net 14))
 (segment (start 124.6451 128.8) (end 123.5201 127.675) (width 0.25) (layer "F.Cu") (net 14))
 (segment (start 134.3445 81.8234) (end 134.3445 77.380149) (width 0.25) (layer "F.Cu") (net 14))
 (segment (start 117.915 136.59) (end 123.463299 136.59) (width 0.25) (layer "F.Cu") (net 14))
 (segment (start 122.9625 75.3) (end 120.8625 77.4) (width 0.25) (layer "F.Cu") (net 14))
 (segment (start 130.49 138.975) (end 131.365 138.1) (width 0.25) (layer "F.Cu") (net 14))
 (segment (start 134.4551 133.3449) (end 134.4551 131.9) (width 0.25) (layer "F.Cu") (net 14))
 (segment (start 132.54 135.26) (end 134.4551 133.3449) (width 0.25) (layer "F.Cu") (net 14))
 (segment (start 132.264351 75.3) (end 122.9625 75.3) (width 0.25) (layer "F.Cu") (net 14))
 (via (at 120.8625 80.4625) (size 0.8) (drill 0.4) (layers "F.Cu" "B.Cu") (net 14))
 (segment (start 115.725 109.725) (end 115.725 82.375) (width 0.25) (layer "B.Cu") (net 14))
 (segment (start 115.725 82.375) (end 116.6426 81.4574) (width 0.25) (layer "B.Cu") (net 14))
 (segment (start 124.6451 128.8) (end 124.6451 118.6451) (width 0.25) (layer "B.Cu") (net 14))
 (segment (start 119.8676 81.4574) (end 120.8625 80.4625) (width 0.25) (layer "B.Cu") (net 14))
 (segment (start 124.6451 118.6451) (end 115.725 109.725) (width 0.25) (layer "B.Cu") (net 14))
 (segment (start 116.6426 81.4574) (end 119.8676 81.4574) (width 0.25) (layer "B.Cu") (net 14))
 (segment (start 119.3 95.2) (end 119.3 89.3329) (width 0.25) (layer "F.Cu") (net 16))
 (segment (start 130.975 120.749695) (end 130.975 104.896927) (width 0.25) (layer "F.Cu") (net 16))
 (segment (start 133.989109 130.775) (end 134.225 130.775) (width 0.25) (layer "F.Cu") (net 16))
 (segment (start 132.625 122.399695) (end 130.975 120.749695) (width 0.25) (layer "F.Cu") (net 16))
 (segment (start 133.989109 130.775) (end 134.921091 130.775) (width 0.25) (layer "F.Cu") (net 16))
 (segment (start 122.558467 95.9) (end 120 95.9) (width 0.25) (layer "F.Cu") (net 16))
 (segment (start 134.225 130.775) (end 135.5801 129.4199) (width 0.25) (layer "F.Cu") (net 16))
 (segment (start 135.5801 131.434009) (end 135.5801 134.7599) (width 0.25) (layer "F.Cu") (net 16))
 (segment (start 120 95.9) (end 119.3 95.2) (width 0.25) (layer "F.Cu") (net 16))
 (segment (start 135.5801 134.7599) (end 132.54 137.8) (width 0.25) (layer "F.Cu") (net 16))
 (segment (start 127.5101 131.225) (end 133.539109 131.225) (width 0.25) (layer "F.Cu") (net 16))
 (segment (start 134.921091 130.775) (end 135.5801 131.434009) (width 0.25) (layer "F.Cu") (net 16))
 (segment (start 126.8351 131.9) (end 127.5101 131.225) (width 0.25) (layer "F.Cu") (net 16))
 (segment (start 135.5801 129.4199) (end 135.5801 125.743704) (width 0.25) (layer "F.Cu") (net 16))
 (segment (start 119.3 89.3329) (end 117.9575 87.9904) (width 0.25) (layer "F.Cu") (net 16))
 (segment (start 133.539109 131.225) (end 133.989109 130.775) (width 0.25) (layer "F.Cu") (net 16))
 (segment (start 130.975 104.896927) (end 126.3103 100.232228) (width 0.25) (layer "F.Cu") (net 16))
 (segment (start 132.625 122.788604) (end 132.625 122.399695) (width 0.25) (layer "F.Cu") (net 16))
 (segment (start 135.5801 125.743704) (end 132.625 122.788604) (width 0.25) (layer "F.Cu") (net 16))
 (segment (start 126.3103 99.651833) (end 122.558467 95.9) (width 0.25) (layer "F.Cu") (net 16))
 (segment (start 126.3103 100.232228) (end 126.3103 99.651833) (width 0.25) (layer "F.Cu") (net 16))
 (segment (start 124.5 135.7) (end 124.5 134.6) (width 0.25) (layer "F.Cu") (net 15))
 (segment (start 116.95 134.05) (end 115.9 133) (width 0.25) (layer "F.Cu") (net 15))
 (segment (start 115.4 93.0879) (end 117.9575 90.5304) (width 0.25) (layer "F.Cu") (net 15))
 (segment (start 123.95 134.05) (end 116.95 134.05) (width 0.25) (layer "F.Cu") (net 15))
 (segment (start 125.2 136.4) (end 124.5 135.7) (width 0.25) (layer "F.Cu") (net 15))
 (segment (start 128.6 136.4) (end 125.2 136.4) (width 0.25) (layer "F.Cu") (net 15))
 (segment (start 115.9 129.9251) (end 117.0251 128.8) (width 0.25) (layer "F.Cu") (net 15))
 (segment (start 130 137.8) (end 128.6 136.4) (width 0.25) (layer "F.Cu") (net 15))
 (segment (start 117 123.2) (end 115.4 121.6) (width 0.25) (layer "F.Cu") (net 15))
 (segment (start 115.4 121.6) (end 115.4 93.0879) (width 0.25) (layer "F.Cu") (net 15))
 (segment (start 124.5 134.6) (end 123.95 134.05) (width 0.25) (layer "F.Cu") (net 15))
 (segment (start 115.9 133) (end 115.9 129.9251) (width 0.25) (layer "F.Cu") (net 15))
 (via (at 117 123.2) (size 0.8) (drill 0.4) (layers "F.Cu" "B.Cu") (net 15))
 (segment (start 117 123.2) (end 117.0251 123.2251) (width 0.25) (layer "B.Cu") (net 15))
 (segment (start 117.0251 123.2251) (end 117.0251 128.8) (width 0.25) (layer "B.Cu") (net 15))
 (segment (start 125.1375 77.4) (end 127.1 77.4) (width 0.25) (layer "F.Cu") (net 13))
 (segment (start 127.1 77.4) (end 130.2871 77.4) (width 0.25) (layer "F.Cu") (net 13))
 (segment (start 130.2871 77.4) (end 133.2575 80.3704) (width 0.25) (layer "F.Cu") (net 13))
 (via (at 127.1 77.4) (size 0.8) (drill 0.4) (layers "F.Cu" "B.Cu") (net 13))
 (segment (start 130.425 87.999695) (end 124.5 82.074695) (width 0.25) (layer "B.Cu") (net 13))
 (segment (start 130.9 92.3) (end 130.9 89.075305) (width 0.25) (layer "B.Cu") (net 13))
 (segment (start 130.9 89.075305) (end 130.425 88.600305) (width 0.25) (layer "B.Cu") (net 13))
 (segment (start 124.5 82.074695) (end 124.5 80) (width 0.25) (layer "B.Cu") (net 13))
 (segment (start 135.3975 96.7975) (end 130.9 92.3) (width 0.25) (layer "B.Cu") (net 13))
 (segment (start 135.3975 122.639158) (end 135.3975 96.7975) (width 0.25) (layer "B.Cu") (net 13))
 (segment (start 130.425 88.600305) (end 130.425 87.999695) (width 0.25) (layer "B.Cu") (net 13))
 (segment (start 130 128.036658) (end 135.3975 122.639158) (width 0.25) (layer "B.Cu") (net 13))
 (segment (start 130 135.26) (end 130 128.036658) (width 0.25) (layer "B.Cu") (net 13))
 (segment (start 124.5 80) (end 127.1 77.4) (width 0.25) (layer "B.Cu") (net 13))
 (segment (start 121.6 100.3) (end 119.55 102.35) (width 0.25) (layer "F.Cu") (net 3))
 (segment (start 119.55 118.15) (end 120 118.6) (width 0.25) (layer "F.Cu") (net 3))
 (segment (start 119.55 118.1) (end 119.55 118.15) (width 0.25) (layer "F.Cu") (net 3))
 (segment (start 119.55 102.35) (end 119.55 118.1) (width 0.25) (layer "F.Cu") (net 3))
 (via (at 120 118.6) (size 0.8) (drill 0.4) (layers "F.Cu" "B.Cu") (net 3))
 (via (at 121.6 100.3) (size 0.8) (drill 0.4) (layers "F.Cu" "B.Cu") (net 3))
 (segment (start 119.05 119.55) (end 119.05 135.075) (width 0.25) (layer "B.Cu") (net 3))
 (segment (start 123.125 98.775) (end 121.6 100.3) (width 0.25) (layer "B.Cu") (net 3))
 (segment (start 123.125 88.0779) (end 123.125 98.775) (width 0.25) (layer "B.Cu") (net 3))
 (segment (start 120 118.6) (end 119.05 119.55) (width 0.25) (layer "B.Cu") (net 3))
 (segment (start 117.9575 82.9104) (end 123.125 88.0779) (width 0.25) (layer "B.Cu") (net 3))
 (segment (start 119.05 135.075) (end 118.9 135.225) (width 0.25) (layer "B.Cu") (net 3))
 (segment (start 119.1 100.6) (end 119.1 118.1) (width 0.25) (layer "F.Cu") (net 4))
 (segment (start 119.1 118.1) (end 118.6 118.6) (width 0.25) (layer "F.Cu") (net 4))
 (segment (start 118.6 118.6) (end 118.7 118.5) (width 0.25) (layer "F.Cu") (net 4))
 (via (at 119.1 100.6) (size 0.8) (drill 0.4) (layers "F.Cu" "B.Cu") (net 4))
 (via (at 118.6 118.6) (size 0.8) (drill 0.4) (layers "F.Cu" "B.Cu") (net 4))
 (segment (start 118.9 137.765) (end 117.725 136.59) (width 0.25) (layer "B.Cu") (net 4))
 (segment (start 119.055 100.555) (end 119.055 97.159745) (width 0.25) (layer "B.Cu") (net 4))
 (segment (start 118.6 132.9) (end 118.6 118.6) (width 0.25) (layer "B.Cu") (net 4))
 (segment (start 119.1 100.6) (end 119.055 100.555) (width 0.25) (layer "B.Cu") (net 4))
 (segment (start 117.725 136.59) (end 117.725 133.775) (width 0.25) (layer "B.Cu") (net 4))
 (segment (start 119.055 97.159745) (end 116.5 94.604745) (width 0.25) (layer "B.Cu") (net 4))
 (segment (start 117.725 133.775) (end 118.6 132.9) (width 0.25) (layer "B.Cu") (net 4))
 (segment (start 116.5 94.604745) (end 116.5 86.9079) (width 0.25) (layer "B.Cu") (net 4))
 (segment (start 116.5 86.9079) (end 117.9575 85.4504) (width 0.25) (layer "B.Cu") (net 4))
 (segment (start 126.800001 82.600001) (end 128.7982 82.600001) (width 0.25) (layer "F.Cu") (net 6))
 (segment (start 126 81.8) (end 126.800001 82.600001) (width 0.25) (layer "F.Cu") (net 6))
 (via (at 126 81.8) (size 0.8) (drill 0.4) (layers "F.Cu" "B.Cu") (free) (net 6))
 (segment (start 130.875 87.813299) (end 130.875 87.9904) (width 0.25) (layer "B.Cu") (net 6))
 (segment (start 126 82.938299) (end 130.875 87.813299) (width 0.25) (layer "B.Cu") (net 6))
 (segment (start 126 81.8) (end 126 82.938299) (width 0.25) (layer "B.Cu") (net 6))
 (segment (start 130.875 87.9904) (end 133.2575 87.9904) (width 0.25) (layer "B.Cu") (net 6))
 (segment (start 126 80.6) (end 127.500002 82.100002) (width 0.25) (layer "F.Cu") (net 5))
 (segment (start 127.500002 82.100002) (end 128.7982 82.100002) (width 0.25) (layer "F.Cu") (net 5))
 (via (at 126 80.6) (size 0.8) (drill 0.4) (layers "F.Cu" "B.Cu") (free) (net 5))
 (segment (start 129.148497 85.4504) (end 133.2575 85.4504) (width 0.25) (layer "B.Cu") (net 5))
 (segment (start 126.725 81.325) (end 126.725 83.026903) (width 0.25) (layer "B.Cu") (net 5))
 (segment (start 126 80.6) (end 126.725 81.325) (width 0.25) (layer "B.Cu") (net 5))
 (segment (start 126.725 83.026903) (end 129.148497 85.4504) (width 0.25) (layer "B.Cu") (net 5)))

